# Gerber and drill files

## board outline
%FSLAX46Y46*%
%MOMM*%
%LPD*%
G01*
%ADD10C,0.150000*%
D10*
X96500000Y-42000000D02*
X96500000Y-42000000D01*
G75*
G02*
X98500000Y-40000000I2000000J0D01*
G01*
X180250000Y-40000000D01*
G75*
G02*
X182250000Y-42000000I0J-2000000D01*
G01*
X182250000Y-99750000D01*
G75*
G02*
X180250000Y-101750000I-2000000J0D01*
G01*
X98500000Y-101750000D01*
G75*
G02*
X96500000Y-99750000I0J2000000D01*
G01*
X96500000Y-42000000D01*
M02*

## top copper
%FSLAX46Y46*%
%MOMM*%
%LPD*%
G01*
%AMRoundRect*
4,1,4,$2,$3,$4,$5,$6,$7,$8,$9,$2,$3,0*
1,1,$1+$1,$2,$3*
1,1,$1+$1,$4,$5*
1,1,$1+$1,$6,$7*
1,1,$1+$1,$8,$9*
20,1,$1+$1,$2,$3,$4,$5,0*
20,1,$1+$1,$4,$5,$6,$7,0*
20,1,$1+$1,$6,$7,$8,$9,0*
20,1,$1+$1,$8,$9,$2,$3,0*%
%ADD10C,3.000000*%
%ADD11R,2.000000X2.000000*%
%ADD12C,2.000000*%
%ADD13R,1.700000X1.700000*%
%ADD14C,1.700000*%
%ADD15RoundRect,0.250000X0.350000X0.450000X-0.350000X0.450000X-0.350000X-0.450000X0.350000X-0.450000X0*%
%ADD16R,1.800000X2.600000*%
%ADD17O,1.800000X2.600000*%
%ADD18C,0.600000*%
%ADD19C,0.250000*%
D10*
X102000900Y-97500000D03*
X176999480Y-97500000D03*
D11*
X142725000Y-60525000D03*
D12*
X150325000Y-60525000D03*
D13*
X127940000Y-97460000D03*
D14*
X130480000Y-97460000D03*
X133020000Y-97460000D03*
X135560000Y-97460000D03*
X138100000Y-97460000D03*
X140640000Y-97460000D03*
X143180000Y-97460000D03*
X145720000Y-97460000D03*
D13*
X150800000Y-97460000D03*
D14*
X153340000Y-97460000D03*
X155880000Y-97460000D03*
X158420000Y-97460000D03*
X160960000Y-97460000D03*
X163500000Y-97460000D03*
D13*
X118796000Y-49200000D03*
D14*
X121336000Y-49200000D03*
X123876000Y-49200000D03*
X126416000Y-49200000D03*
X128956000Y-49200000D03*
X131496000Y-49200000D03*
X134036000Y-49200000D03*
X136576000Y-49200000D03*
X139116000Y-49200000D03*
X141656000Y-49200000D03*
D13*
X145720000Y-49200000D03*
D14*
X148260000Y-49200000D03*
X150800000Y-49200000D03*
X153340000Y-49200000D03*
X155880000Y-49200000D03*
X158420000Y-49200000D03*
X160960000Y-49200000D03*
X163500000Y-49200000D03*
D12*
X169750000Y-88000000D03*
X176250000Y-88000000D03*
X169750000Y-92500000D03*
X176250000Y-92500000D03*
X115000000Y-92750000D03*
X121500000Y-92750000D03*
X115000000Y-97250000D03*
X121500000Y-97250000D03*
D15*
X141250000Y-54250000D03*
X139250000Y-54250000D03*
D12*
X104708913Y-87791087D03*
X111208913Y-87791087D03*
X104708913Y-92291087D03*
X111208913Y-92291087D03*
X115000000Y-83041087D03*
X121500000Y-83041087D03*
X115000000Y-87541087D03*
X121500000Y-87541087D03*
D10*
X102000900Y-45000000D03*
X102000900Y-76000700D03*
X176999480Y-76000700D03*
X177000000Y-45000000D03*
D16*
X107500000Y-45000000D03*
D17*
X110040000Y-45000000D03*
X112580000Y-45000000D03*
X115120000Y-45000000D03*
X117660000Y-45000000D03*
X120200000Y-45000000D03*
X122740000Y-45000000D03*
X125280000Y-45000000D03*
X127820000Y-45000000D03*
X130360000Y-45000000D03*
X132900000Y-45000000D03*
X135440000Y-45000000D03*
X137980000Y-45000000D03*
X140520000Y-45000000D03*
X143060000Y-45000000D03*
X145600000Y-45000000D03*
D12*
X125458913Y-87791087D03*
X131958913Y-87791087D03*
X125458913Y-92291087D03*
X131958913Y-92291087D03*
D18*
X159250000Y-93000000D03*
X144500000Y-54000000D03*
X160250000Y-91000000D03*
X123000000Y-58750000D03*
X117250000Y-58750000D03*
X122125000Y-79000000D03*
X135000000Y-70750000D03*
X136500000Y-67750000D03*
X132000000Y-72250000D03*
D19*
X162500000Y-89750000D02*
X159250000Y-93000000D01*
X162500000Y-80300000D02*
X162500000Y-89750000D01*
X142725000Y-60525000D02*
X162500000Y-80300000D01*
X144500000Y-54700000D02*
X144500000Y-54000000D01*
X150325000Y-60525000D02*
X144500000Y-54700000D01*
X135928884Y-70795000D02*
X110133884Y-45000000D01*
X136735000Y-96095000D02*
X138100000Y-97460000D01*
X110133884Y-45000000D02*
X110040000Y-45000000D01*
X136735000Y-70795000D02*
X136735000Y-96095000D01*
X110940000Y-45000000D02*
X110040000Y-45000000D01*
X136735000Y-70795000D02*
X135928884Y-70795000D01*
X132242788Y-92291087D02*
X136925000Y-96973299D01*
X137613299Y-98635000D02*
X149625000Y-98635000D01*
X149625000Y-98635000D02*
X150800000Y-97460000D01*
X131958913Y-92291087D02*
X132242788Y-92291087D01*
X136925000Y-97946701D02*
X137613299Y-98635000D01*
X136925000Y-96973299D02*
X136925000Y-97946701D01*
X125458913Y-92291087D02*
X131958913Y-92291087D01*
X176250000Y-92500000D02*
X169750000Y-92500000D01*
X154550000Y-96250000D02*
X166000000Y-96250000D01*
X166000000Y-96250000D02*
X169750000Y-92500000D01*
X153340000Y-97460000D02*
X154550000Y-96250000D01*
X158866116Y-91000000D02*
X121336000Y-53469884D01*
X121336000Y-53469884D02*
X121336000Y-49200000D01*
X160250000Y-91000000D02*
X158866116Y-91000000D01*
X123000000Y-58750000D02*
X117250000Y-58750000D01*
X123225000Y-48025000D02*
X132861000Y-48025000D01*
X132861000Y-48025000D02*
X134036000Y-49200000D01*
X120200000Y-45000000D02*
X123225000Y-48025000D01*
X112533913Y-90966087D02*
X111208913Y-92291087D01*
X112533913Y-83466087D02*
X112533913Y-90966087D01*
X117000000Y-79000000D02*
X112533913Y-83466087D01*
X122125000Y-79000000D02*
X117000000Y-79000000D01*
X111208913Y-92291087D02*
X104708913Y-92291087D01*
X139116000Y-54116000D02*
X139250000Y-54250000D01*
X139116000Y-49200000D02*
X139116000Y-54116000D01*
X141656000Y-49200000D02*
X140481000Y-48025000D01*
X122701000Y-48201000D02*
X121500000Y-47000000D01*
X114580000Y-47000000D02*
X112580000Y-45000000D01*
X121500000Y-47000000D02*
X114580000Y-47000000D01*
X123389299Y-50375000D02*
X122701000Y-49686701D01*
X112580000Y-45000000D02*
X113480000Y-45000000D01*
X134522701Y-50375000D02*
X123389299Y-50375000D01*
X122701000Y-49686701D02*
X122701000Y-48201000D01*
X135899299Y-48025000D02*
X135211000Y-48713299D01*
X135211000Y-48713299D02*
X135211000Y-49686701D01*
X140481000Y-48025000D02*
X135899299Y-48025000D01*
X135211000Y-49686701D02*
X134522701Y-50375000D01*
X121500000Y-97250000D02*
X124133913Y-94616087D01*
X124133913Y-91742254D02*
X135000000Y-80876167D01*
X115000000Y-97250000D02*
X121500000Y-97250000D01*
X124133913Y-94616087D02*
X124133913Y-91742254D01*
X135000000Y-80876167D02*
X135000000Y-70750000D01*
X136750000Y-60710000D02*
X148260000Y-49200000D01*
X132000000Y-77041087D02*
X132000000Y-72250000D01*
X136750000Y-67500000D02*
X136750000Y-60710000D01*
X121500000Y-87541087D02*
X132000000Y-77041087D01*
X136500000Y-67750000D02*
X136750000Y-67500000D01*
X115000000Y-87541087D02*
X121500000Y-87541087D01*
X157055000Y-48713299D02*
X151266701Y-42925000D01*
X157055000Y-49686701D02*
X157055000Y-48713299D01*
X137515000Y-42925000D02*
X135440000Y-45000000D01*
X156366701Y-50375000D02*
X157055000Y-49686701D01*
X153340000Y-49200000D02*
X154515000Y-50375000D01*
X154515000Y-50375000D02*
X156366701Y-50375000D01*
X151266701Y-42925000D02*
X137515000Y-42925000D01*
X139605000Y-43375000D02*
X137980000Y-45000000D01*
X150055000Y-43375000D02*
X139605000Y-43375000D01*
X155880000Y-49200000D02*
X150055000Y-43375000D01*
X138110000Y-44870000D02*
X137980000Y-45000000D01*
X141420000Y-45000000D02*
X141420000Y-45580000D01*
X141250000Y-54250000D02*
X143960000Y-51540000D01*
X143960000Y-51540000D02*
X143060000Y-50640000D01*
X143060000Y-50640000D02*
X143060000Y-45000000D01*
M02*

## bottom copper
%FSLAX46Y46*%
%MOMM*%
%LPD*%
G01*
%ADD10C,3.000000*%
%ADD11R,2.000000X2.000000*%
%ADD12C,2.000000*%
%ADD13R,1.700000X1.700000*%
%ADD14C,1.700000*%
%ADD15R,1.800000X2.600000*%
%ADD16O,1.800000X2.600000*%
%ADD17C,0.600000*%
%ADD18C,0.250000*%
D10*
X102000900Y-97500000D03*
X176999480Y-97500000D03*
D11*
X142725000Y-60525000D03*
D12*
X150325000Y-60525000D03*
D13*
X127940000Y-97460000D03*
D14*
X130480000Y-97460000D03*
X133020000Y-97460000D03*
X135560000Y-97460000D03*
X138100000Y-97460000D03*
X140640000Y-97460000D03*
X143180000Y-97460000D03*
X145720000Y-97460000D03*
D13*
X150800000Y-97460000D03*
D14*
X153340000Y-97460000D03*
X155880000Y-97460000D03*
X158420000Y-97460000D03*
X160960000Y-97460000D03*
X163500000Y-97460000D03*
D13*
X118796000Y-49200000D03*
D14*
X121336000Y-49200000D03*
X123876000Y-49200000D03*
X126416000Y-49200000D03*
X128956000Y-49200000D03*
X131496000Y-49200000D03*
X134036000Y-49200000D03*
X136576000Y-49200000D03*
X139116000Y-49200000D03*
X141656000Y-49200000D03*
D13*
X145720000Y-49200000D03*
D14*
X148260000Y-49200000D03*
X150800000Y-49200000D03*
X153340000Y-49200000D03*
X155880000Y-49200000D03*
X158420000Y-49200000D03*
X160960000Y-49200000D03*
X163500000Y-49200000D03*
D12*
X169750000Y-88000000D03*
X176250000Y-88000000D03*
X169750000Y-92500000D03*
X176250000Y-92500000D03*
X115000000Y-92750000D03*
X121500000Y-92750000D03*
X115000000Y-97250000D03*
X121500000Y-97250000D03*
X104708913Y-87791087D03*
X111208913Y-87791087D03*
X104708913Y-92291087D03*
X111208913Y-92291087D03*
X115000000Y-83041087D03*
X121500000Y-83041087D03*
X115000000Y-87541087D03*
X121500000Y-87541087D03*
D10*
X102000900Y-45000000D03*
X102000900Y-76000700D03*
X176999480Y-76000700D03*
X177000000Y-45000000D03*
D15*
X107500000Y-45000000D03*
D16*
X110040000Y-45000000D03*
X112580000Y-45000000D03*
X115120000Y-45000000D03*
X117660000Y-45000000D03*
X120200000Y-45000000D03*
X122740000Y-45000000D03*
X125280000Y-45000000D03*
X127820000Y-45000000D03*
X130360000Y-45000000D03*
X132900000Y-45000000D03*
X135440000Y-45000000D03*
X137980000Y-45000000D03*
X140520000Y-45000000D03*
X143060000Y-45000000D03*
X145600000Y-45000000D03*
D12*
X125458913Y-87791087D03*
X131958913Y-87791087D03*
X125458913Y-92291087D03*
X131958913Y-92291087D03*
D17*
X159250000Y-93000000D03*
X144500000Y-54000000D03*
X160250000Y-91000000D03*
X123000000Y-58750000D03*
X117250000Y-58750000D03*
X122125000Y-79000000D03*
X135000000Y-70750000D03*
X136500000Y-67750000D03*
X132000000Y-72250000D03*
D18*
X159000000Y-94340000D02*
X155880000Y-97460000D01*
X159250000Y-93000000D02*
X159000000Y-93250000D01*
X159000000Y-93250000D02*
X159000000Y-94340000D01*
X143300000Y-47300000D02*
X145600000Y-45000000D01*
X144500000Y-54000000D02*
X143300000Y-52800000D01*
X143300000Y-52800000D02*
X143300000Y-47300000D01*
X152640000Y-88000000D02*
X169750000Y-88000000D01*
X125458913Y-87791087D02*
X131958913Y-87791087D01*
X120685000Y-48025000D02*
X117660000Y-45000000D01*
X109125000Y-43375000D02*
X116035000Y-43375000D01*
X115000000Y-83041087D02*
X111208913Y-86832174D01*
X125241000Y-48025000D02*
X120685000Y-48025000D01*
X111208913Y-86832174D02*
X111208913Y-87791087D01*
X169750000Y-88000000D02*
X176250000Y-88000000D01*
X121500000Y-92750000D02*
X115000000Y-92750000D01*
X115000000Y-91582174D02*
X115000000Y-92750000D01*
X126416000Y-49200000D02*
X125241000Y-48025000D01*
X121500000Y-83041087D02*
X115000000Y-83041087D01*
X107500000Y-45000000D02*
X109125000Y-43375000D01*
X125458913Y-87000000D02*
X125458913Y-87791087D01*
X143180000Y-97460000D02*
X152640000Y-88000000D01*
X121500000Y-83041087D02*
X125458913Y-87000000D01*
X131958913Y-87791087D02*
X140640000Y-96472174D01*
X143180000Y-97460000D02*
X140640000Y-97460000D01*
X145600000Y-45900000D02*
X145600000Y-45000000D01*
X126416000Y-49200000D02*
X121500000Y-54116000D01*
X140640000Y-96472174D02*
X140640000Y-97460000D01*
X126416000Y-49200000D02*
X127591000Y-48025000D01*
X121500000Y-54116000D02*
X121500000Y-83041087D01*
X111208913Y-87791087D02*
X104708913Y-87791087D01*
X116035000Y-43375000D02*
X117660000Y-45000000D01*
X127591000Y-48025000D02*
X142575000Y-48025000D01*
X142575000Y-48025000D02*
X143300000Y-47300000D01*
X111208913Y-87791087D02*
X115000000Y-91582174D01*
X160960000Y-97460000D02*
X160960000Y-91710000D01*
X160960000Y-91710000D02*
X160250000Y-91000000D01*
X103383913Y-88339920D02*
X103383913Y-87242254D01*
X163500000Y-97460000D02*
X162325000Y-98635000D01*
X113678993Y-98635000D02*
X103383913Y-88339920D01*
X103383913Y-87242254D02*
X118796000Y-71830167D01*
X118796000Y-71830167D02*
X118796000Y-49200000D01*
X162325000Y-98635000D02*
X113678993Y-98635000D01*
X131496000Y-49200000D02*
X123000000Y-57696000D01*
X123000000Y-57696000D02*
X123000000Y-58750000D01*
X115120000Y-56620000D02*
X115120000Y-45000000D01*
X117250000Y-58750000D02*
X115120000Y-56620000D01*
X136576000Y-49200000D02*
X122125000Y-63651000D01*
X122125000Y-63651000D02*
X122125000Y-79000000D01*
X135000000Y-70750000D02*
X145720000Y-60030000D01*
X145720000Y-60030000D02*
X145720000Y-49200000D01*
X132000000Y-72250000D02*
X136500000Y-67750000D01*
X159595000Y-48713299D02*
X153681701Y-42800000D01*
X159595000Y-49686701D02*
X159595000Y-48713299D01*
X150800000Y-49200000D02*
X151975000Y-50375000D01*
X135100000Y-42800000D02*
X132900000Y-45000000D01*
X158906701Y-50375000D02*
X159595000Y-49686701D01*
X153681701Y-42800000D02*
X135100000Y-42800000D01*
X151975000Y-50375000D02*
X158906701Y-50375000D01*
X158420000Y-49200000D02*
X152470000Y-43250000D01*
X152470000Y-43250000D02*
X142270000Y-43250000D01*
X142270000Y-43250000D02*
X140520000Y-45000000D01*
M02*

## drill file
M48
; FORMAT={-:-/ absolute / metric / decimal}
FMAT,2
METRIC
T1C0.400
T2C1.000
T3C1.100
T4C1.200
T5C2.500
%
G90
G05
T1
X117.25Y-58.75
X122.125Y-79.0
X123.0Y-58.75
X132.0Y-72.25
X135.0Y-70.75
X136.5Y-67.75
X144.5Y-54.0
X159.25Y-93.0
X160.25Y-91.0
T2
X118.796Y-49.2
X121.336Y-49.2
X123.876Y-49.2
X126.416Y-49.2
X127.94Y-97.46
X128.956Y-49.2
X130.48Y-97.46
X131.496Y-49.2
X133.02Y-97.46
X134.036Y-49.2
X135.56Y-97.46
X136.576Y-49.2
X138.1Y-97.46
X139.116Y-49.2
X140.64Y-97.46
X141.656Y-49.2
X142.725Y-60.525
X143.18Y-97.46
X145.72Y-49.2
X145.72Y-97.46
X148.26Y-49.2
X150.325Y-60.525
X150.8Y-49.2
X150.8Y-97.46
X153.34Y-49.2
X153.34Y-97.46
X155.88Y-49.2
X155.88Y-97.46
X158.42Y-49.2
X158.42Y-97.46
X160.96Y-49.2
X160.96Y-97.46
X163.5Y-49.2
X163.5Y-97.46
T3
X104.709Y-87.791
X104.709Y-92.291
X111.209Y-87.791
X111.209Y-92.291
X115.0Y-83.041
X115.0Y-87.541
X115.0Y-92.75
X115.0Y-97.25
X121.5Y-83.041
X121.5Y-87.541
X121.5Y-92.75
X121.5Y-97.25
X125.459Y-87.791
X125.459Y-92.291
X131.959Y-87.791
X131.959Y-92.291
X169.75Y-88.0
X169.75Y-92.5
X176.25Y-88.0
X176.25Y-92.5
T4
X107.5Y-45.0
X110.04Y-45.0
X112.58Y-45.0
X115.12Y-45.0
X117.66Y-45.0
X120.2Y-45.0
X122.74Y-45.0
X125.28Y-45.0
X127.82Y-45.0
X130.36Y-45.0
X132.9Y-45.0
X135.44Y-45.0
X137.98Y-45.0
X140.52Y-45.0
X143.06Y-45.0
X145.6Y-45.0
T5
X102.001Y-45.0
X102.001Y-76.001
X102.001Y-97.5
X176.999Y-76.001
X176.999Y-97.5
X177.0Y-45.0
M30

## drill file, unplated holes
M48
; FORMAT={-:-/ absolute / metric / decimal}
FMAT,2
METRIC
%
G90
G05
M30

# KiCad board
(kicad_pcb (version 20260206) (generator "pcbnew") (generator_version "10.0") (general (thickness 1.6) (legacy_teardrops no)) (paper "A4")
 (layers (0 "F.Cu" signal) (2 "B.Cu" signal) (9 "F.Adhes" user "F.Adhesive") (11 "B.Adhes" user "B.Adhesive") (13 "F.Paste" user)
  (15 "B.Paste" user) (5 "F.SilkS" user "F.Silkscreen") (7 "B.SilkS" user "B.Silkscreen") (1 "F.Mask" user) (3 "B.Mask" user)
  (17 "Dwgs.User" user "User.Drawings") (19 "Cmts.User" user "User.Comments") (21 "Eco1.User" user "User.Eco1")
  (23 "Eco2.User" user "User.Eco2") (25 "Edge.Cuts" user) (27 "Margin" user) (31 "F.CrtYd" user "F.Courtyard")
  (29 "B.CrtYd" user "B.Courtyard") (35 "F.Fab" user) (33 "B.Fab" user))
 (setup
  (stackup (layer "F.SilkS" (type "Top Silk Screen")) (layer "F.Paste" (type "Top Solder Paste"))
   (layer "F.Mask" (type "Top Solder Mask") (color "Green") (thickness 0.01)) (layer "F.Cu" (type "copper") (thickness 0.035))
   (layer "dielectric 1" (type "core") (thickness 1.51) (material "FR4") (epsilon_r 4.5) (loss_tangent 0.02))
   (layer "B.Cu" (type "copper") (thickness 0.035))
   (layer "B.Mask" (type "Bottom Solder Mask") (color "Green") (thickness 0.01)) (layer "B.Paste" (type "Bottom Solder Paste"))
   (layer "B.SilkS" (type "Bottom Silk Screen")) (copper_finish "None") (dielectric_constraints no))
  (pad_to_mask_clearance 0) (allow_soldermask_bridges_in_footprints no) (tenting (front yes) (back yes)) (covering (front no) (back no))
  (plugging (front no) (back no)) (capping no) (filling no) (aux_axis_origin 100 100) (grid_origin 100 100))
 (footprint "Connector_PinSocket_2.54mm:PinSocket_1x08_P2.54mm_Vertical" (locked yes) (layer "F.Cu") (at 127.94 97.46 90)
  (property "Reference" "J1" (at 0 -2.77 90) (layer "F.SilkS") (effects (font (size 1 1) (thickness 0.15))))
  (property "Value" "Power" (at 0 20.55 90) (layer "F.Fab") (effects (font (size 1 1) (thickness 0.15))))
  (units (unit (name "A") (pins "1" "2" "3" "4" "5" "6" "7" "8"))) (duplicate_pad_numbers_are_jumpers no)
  (pad "1" thru_hole rect (at 0 0 90) (size 1.7 1.7) (drill 1) (layers "*.Cu" "*.Mask") (remove_unused_layers no)
   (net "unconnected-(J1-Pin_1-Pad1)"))
  (pad "2" thru_hole circle (at 0 2.54 90) (size 1.7 1.7) (drill 1) (layers "*.Cu" "*.Mask") (remove_unused_layers no) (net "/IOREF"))
  (pad "3" thru_hole circle (at 0 5.08 90) (size 1.7 1.7) (drill 1) (layers "*.Cu" "*.Mask") (remove_unused_layers no) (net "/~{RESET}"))
  (pad "4" thru_hole circle (at 0 7.62 90) (size 1.7 1.7) (drill 1) (layers "*.Cu" "*.Mask") (remove_unused_layers no) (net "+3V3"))
  (pad "5" thru_hole circle (at 0 10.16 90) (size 1.7 1.7) (drill 1) (layers "*.Cu" "*.Mask") (remove_unused_layers no) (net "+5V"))
  (pad "6" thru_hole circle (at 0 12.7 90) (size 1.7 1.7) (drill 1) (layers "*.Cu" "*.Mask") (remove_unused_layers no) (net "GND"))
  (pad "7" thru_hole circle (at 0 15.24 90) (size 1.7 1.7) (drill 1) (layers "*.Cu" "*.Mask") (remove_unused_layers no) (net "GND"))
  (pad "8" thru_hole circle (at 0 17.78 90) (size 1.7 1.7) (drill 1) (layers "*.Cu" "*.Mask") (remove_unused_layers no) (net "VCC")))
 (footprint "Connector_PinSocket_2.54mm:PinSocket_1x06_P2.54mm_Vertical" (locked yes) (layer "F.Cu") (at 150.8 97.46 90)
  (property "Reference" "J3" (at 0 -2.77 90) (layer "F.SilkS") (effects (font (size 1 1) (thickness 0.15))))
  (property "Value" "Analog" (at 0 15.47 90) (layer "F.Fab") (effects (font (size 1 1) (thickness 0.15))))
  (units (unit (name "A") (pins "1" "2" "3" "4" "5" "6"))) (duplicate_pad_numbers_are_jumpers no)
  (pad "1" thru_hole rect (at 0 0 90) (size 1.7 1.7) (drill 1) (layers "*.Cu" "*.Mask") (remove_unused_layers no) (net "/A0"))
  (pad "2" thru_hole circle (at 0 2.54 90) (size 1.7 1.7) (drill 1) (layers "*.Cu" "*.Mask") (remove_unused_layers no) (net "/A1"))
  (pad "3" thru_hole circle (at 0 5.08 90) (size 1.7 1.7) (drill 1) (layers "*.Cu" "*.Mask") (remove_unused_layers no) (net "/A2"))
  (pad "4" thru_hole circle (at 0 7.62 90) (size 1.7 1.7) (drill 1) (layers "*.Cu" "*.Mask") (remove_unused_layers no) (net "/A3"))
  (pad "5" thru_hole circle (at 0 10.16 90) (size 1.7 1.7) (drill 1) (layers "*.Cu" "*.Mask") (remove_unused_layers no)
   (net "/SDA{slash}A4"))
  (pad "6" thru_hole circle (at 0 12.7 90) (size 1.7 1.7) (drill 1) (layers "*.Cu" "*.Mask") (remove_unused_layers no) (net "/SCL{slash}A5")))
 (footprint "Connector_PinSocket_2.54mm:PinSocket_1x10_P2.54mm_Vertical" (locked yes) (layer "F.Cu") (at 118.796 49.2 90)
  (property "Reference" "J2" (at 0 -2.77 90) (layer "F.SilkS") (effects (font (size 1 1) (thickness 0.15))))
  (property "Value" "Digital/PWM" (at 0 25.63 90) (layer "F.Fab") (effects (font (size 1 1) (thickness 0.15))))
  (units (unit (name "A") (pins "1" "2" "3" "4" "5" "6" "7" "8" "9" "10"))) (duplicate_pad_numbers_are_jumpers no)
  (pad "1" thru_hole rect (at 0 0 90) (size 1.7 1.7) (drill 1) (layers "*.Cu" "*.Mask") (remove_unused_layers no) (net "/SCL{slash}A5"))
  (pad "2" thru_hole circle (at 0 2.54 90) (size 1.7 1.7) (drill 1) (layers "*.Cu" "*.Mask") (remove_unused_layers no) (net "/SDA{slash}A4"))
  (pad "3" thru_hole circle (at 0 5.08 90) (size 1.7 1.7) (drill 1) (layers "*.Cu" "*.Mask") (remove_unused_layers no) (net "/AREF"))
  (pad "4" thru_hole circle (at 0 7.62 90) (size 1.7 1.7) (drill 1) (layers "*.Cu" "*.Mask") (remove_unused_layers no) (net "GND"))
  (pad "5" thru_hole circle (at 0 10.16 90) (size 1.7 1.7) (drill 1) (layers "*.Cu" "*.Mask") (remove_unused_layers no) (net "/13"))
  (pad "6" thru_hole circle (at 0 12.7 90) (size 1.7 1.7) (drill 1) (layers "*.Cu" "*.Mask") (remove_unused_layers no) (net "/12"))
  (pad "7" thru_hole circle (at 0 15.24 90) (size 1.7 1.7) (drill 1) (layers "*.Cu" "*.Mask") (remove_unused_layers no) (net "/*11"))
  (pad "8" thru_hole circle (at 0 17.78 90) (size 1.7 1.7) (drill 1) (layers "*.Cu" "*.Mask") (remove_unused_layers no) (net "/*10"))
  (pad "9" thru_hole circle (at 0 20.32 90) (size 1.7 1.7) (drill 1) (layers "*.Cu" "*.Mask") (remove_unused_layers no) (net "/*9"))
  (pad "10" thru_hole circle (at 0 22.86 90) (size 1.7 1.7) (drill 1) (layers "*.Cu" "*.Mask") (remove_unused_layers no) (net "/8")))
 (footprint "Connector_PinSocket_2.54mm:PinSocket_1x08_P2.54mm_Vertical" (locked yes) (layer "F.Cu") (at 145.72 49.2 90)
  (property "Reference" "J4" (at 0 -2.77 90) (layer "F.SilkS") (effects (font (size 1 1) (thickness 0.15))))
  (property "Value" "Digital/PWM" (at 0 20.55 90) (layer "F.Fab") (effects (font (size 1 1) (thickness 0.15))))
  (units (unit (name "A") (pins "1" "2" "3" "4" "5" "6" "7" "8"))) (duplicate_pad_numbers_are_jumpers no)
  (pad "1" thru_hole rect (at 0 0 90) (size 1.7 1.7) (drill 1) (layers "*.Cu" "*.Mask") (remove_unused_layers no) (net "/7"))
  (pad "2" thru_hole circle (at 0 2.54 90) (size 1.7 1.7) (drill 1) (layers "*.Cu" "*.Mask") (remove_unused_layers no) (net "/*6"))
  (pad "3" thru_hole circle (at 0 5.08 90) (size 1.7 1.7) (drill 1) (layers "*.Cu" "*.Mask") (remove_unused_layers no) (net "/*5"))
  (pad "4" thru_hole circle (at 0 7.62 90) (size 1.7 1.7) (drill 1) (layers "*.Cu" "*.Mask") (remove_unused_layers no) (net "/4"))
  (pad "5" thru_hole circle (at 0 10.16 90) (size 1.7 1.7) (drill 1) (layers "*.Cu" "*.Mask") (remove_unused_layers no) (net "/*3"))
  (pad "6" thru_hole circle (at 0 12.7 90) (size 1.7 1.7) (drill 1) (layers "*.Cu" "*.Mask") (remove_unused_layers no) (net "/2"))
  (pad "7" thru_hole circle (at 0 15.24 90) (size 1.7 1.7) (drill 1) (layers "*.Cu" "*.Mask") (remove_unused_layers no) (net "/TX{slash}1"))
  (pad "8" thru_hole circle (at 0 17.78 90) (size 1.7 1.7) (drill 1) (layers "*.Cu" "*.Mask") (remove_unused_layers no) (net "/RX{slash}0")))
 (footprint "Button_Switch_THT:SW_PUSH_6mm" (layer "F.Cu") (at 169.75 88)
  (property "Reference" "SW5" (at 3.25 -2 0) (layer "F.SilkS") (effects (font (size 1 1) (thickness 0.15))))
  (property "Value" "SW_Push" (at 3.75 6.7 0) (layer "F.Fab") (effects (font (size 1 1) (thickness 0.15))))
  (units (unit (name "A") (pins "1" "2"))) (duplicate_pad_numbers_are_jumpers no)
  (pad "1" thru_hole circle (at 0 0 90) (size 2 2) (drill 1.1) (layers "*.Cu" "*.Mask") (remove_unused_layers no) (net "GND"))
  (pad "1" thru_hole circle (at 6.5 0 90) (size 2 2) (drill 1.1) (layers "*.Cu" "*.Mask") (remove_unused_layers no) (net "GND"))
  (pad "2" thru_hole circle (at 0 4.5 90) (size 2 2) (drill 1.1) (layers "*.Cu" "*.Mask") (remove_unused_layers no) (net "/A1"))
  (pad "2" thru_hole circle (at 6.5 4.5 90) (size 2 2) (drill 1.1) (layers "*.Cu" "*.Mask") (remove_unused_layers no) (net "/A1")))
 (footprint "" (layer "F.Cu") (at 176.99948 97.5)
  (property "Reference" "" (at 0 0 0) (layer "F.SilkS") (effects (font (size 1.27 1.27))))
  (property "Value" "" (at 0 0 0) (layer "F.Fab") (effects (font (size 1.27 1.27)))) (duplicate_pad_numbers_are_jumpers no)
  (pad "" thru_hole circle (at 0 0) (size 3 3) (drill 2.5) (layers "*.Cu" "*.Mask") (remove_unused_layers no)))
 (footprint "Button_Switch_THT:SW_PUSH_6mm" (layer "F.Cu") (at 115 92.75)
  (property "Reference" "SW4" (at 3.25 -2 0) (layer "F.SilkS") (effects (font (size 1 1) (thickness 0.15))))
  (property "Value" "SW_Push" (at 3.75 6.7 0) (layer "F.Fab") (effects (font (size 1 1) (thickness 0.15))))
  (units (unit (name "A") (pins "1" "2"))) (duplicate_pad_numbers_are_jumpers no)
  (pad "1" thru_hole circle (at 0 0 90) (size 2 2) (drill 1.1) (layers "*.Cu" "*.Mask") (remove_unused_layers no) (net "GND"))
  (pad "1" thru_hole circle (at 6.5 0 90) (size 2 2) (drill 1.1) (layers "*.Cu" "*.Mask") (remove_unused_layers no) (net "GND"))
  (pad "2" thru_hole circle (at 0 4.5 90) (size 2 2) (drill 1.1) (layers "*.Cu" "*.Mask") (remove_unused_layers no) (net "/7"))
  (pad "2" thru_hole circle (at 6.5 4.5 90) (size 2 2) (drill 1.1) (layers "*.Cu" "*.Mask") (remove_unused_layers no) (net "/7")))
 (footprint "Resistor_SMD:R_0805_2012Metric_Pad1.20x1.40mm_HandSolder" (layer "F.Cu") (at 140.25 54.25 180)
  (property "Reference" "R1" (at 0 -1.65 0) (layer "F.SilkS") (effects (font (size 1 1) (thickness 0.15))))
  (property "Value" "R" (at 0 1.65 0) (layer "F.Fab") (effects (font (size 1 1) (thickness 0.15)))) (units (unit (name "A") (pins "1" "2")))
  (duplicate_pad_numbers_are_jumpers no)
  (pad "1" smd roundrect (at -1 0 180) (size 1.2 1.4) (layers "F.Cu" "F.Mask" "F.Paste") (roundrect_rratio 0.208333)
   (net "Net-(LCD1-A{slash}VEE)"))
  (pad "2" smd roundrect (at 1 0 180) (size 1.2 1.4) (layers "F.Cu" "F.Mask" "F.Paste") (roundrect_rratio 0.208333) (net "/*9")))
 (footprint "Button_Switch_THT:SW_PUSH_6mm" (layer "F.Cu") (at 104.708913 87.791087)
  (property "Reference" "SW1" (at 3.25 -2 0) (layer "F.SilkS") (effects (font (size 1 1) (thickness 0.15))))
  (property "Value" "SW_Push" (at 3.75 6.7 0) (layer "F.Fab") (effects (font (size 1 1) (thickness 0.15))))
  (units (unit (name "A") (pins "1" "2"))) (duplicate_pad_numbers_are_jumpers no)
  (pad "1" thru_hole circle (at 0 0 90) (size 2 2) (drill 1.1) (layers "*.Cu" "*.Mask") (remove_unused_layers no) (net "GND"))
  (pad "1" thru_hole circle (at 6.5 0 90) (size 2 2) (drill 1.1) (layers "*.Cu" "*.Mask") (remove_unused_layers no) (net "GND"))
  (pad "2" thru_hole circle (at 0 4.5 90) (size 2 2) (drill 1.1) (layers "*.Cu" "*.Mask") (remove_unused_layers no) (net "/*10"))
  (pad "2" thru_hole circle (at 6.5 4.5 90) (size 2 2) (drill 1.1) (layers "*.Cu" "*.Mask") (remove_unused_layers no) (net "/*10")))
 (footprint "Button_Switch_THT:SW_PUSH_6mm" (layer "F.Cu") (at 115 83.041087)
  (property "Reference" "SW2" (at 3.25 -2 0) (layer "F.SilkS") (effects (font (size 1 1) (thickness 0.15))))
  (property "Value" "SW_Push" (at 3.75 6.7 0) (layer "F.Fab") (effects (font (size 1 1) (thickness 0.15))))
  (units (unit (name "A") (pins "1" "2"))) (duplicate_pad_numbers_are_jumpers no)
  (pad "1" thru_hole circle (at 0 0 90) (size 2 2) (drill 1.1) (layers "*.Cu" "*.Mask") (remove_unused_layers no) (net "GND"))
  (pad "1" thru_hole circle (at 6.5 0 90) (size 2 2) (drill 1.1) (layers "*.Cu" "*.Mask") (remove_unused_layers no) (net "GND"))
  (pad "2" thru_hole circle (at 0 4.5 90) (size 2 2) (drill 1.1) (layers "*.Cu" "*.Mask") (remove_unused_layers no) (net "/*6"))
  (pad "2" thru_hole circle (at 6.5 4.5 90) (size 2 2) (drill 1.1) (layers "*.Cu" "*.Mask") (remove_unused_layers no) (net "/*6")))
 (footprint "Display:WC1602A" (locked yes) (layer "F.Cu") (at 107.5 45)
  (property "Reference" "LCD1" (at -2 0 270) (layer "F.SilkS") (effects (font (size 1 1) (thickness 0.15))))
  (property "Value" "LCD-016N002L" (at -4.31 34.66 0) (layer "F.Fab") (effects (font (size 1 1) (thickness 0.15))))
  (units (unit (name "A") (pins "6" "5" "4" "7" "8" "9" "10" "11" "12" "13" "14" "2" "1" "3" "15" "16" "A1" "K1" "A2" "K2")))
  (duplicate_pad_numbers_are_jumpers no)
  (pad "" thru_hole circle (at -5.4991 0) (size 3 3) (drill 2.5) (layers "*.Cu" "*.Mask") (remove_unused_layers no))
  (pad "" thru_hole circle (at -5.4991 31.0007) (size 3 3) (drill 2.5) (layers "*.Cu" "*.Mask") (remove_unused_layers no))
  (pad "" thru_hole circle (at 69.49948 31.0007) (size 3 3) (drill 2.5) (layers "*.Cu" "*.Mask") (remove_unused_layers no))
  (pad "" thru_hole circle (at 69.5 0) (size 3 3) (drill 2.5) (layers "*.Cu" "*.Mask") (remove_unused_layers no))
  (pad "1" thru_hole rect (at 0 0) (size 1.8 2.6) (drill 1.2) (layers "*.Cu" "*.Mask") (remove_unused_layers no) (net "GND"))
  (pad "2" thru_hole oval (at 2.54 0) (size 1.8 2.6) (drill 1.2) (layers "*.Cu" "*.Mask") (remove_unused_layers no) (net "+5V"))
  (pad "3" thru_hole oval (at 5.08 0) (size 1.8 2.6) (drill 1.2) (layers "*.Cu" "*.Mask") (remove_unused_layers no) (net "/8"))
  (pad "4" thru_hole oval (at 7.62 0) (size 1.8 2.6) (drill 1.2) (layers "*.Cu" "*.Mask") (remove_unused_layers no) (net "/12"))
  (pad "5" thru_hole oval (at 10.16 0) (size 1.8 2.6) (drill 1.2) (layers "*.Cu" "*.Mask") (remove_unused_layers no) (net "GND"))
  (pad "6" thru_hole oval (at 12.7 0) (size 1.8 2.6) (drill 1.2) (layers "*.Cu" "*.Mask") (remove_unused_layers no) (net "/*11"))
  (pad "7" thru_hole oval (at 15.24 0) (size 1.8 2.6) (drill 1.2) (layers "*.Cu" "*.Mask") (remove_unused_layers no)
   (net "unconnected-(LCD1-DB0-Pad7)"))
  (pad "8" thru_hole oval (at 17.78 0) (size 1.8 2.6) (drill 1.2) (layers "*.Cu" "*.Mask") (remove_unused_layers no)
   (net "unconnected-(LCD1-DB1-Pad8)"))
  (pad "9" thru_hole oval (at 20.32 0) (size 1.8 2.6) (drill 1.2) (layers "*.Cu" "*.Mask") (remove_unused_layers no)
   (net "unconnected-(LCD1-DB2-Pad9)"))
  (pad "10" thru_hole oval (at 22.86 0) (size 1.8 2.6) (drill 1.2) (layers "*.Cu" "*.Mask") (remove_unused_layers no)
   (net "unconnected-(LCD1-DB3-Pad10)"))
  (pad "11" thru_hole oval (at 25.4 0) (size 1.8 2.6) (drill 1.2) (layers "*.Cu" "*.Mask") (remove_unused_layers no) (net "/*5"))
  (pad "12" thru_hole oval (at 27.94 0) (size 1.8 2.6) (drill 1.2) (layers "*.Cu" "*.Mask") (remove_unused_layers no) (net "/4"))
  (pad "13" thru_hole oval (at 30.48 0) (size 1.8 2.6) (drill 1.2) (layers "*.Cu" "*.Mask") (remove_unused_layers no) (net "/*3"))
  (pad "14" thru_hole oval (at 33.02 0) (size 1.8 2.6) (drill 1.2) (layers "*.Cu" "*.Mask") (remove_unused_layers no) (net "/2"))
  (pad "15" thru_hole oval (at 35.56 0) (size 1.8 2.6) (drill 1.2) (layers "*.Cu" "*.Mask") (remove_unused_layers no)
   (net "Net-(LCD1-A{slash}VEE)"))
  (pad "16" thru_hole oval (at 38.1 0) (size 1.8 2.6) (drill 1.2) (layers "*.Cu" "*.Mask") (remove_unused_layers no) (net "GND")))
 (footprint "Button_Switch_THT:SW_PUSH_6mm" (layer "F.Cu") (at 125.458913 87.791087)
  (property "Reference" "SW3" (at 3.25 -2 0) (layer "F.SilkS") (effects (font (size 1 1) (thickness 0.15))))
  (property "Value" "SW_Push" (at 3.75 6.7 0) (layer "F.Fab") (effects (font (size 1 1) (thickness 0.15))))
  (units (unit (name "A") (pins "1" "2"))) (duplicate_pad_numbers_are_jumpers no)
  (pad "1" thru_hole circle (at 0 0 90) (size 2 2) (drill 1.1) (layers "*.Cu" "*.Mask") (remove_unused_layers no) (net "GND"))
  (pad "1" thru_hole circle (at 6.5 0 90) (size 2 2) (drill 1.1) (layers "*.Cu" "*.Mask") (remove_unused_layers no) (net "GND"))
  (pad "2" thru_hole circle (at 0 4.5 90) (size 2 2) (drill 1.1) (layers "*.Cu" "*.Mask") (remove_unused_layers no) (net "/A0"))
  (pad "2" thru_hole circle (at 6.5 4.5 90) (size 2 2) (drill 1.1) (layers "*.Cu" "*.Mask") (remove_unused_layers no) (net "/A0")))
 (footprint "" (layer "F.Cu") (at 102.0009 97.5)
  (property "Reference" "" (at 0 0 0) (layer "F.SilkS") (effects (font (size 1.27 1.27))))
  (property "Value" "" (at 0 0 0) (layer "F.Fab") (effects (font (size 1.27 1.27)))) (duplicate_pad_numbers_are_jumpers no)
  (pad "" thru_hole circle (at 0 0) (size 3 3) (drill 2.5) (layers "*.Cu" "*.Mask") (remove_unused_layers no)))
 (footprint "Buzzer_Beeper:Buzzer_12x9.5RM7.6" (layer "F.Cu") (at 142.725 60.525)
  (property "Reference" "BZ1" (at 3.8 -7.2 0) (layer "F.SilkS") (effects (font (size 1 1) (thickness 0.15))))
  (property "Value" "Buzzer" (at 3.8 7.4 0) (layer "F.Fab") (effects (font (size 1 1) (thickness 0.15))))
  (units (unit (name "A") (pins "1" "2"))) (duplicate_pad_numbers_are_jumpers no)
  (pad "1" thru_hole rect (at 0 0) (size 2 2) (drill 1) (layers "*.Cu" "*.Mask") (remove_unused_layers no) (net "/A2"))
  (pad "2" thru_hole circle (at 7.6 0) (size 2 2) (drill 1) (layers "*.Cu" "*.Mask") (remove_unused_layers no) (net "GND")))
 (gr_rect (start 96.5 40) (end 182.25 101.75) (radius 2) (stroke (width 0.15) (type solid)) (fill no) (layer "Edge.Cuts"))
 (segment (start 135.928884 70.795) (end 110.133884 45) (width 0.25) (layer "F.Cu") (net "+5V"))
 (segment (start 136.735 96.095) (end 138.1 97.46) (width 0.25) (layer "F.Cu") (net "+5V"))
 (segment (start 110.133884 45) (end 110.04 45) (width 0.25) (layer "F.Cu") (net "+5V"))
 (segment (start 136.735 70.795) (end 136.735 96.095) (width 0.25) (layer "F.Cu") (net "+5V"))
 (segment (start 110.94 45) (end 110.04 45) (width 0.25) (layer "F.Cu") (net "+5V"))
 (segment (start 136.735 70.795) (end 135.928884 70.795) (width 0.25) (layer "F.Cu") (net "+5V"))
 (segment (start 144.5 54.7) (end 144.5 54) (width 0.25) (layer "F.Cu") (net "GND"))
 (segment (start 150.325 60.525) (end 144.5 54.7) (width 0.25) (layer "F.Cu") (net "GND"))
 (via (at 144.5 54) (size 0.6) (drill 0.4) (layers "F.Cu" "B.Cu") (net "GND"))
 (segment (start 143.3 47.3) (end 145.6 45) (width 0.25) (layer "B.Cu") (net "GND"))
 (segment (start 152.64 88) (end 169.75 88) (width 0.25) (layer "B.Cu") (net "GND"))
 (segment (start 125.458913 87.791087) (end 131.958913 87.791087) (width 0.25) (layer "B.Cu") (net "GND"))
 (segment (start 120.685 48.025) (end 117.66 45) (width 0.25) (layer "B.Cu") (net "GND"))
 (segment (start 109.125 43.375) (end 116.035 43.375) (width 0.25) (layer "B.Cu") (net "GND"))
 (segment (start 115 83.041087) (end 111.208913 86.832174) (width 0.25) (layer "B.Cu") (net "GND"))
 (segment (start 125.241 48.025) (end 120.685 48.025) (width 0.25) (layer "B.Cu") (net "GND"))
 (segment (start 111.208913 86.832174) (end 111.208913 87.791087) (width 0.25) (layer "B.Cu") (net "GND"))
 (segment (start 169.75 88) (end 176.25 88) (width 0.25) (layer "B.Cu") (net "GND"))
 (segment (start 121.5 92.75) (end 115 92.75) (width 0.25) (layer "B.Cu") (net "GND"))
 (segment (start 115 91.582174) (end 115 92.75) (width 0.25) (layer "B.Cu") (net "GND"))
 (segment (start 126.416 49.2) (end 125.241 48.025) (width 0.25) (layer "B.Cu") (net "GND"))
 (segment (start 121.5 83.041087) (end 115 83.041087) (width 0.25) (layer "B.Cu") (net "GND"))
 (segment (start 144.5 54) (end 143.3 52.8) (width 0.25) (layer "B.Cu") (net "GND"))
 (segment (start 107.5 45) (end 109.125 43.375) (width 0.25) (layer "B.Cu") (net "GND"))
 (segment (start 125.458913 87) (end 125.458913 87.791087) (width 0.25) (layer "B.Cu") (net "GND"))
 (segment (start 143.18 97.46) (end 152.64 88) (width 0.25) (layer "B.Cu") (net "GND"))
 (segment (start 121.5 83.041087) (end 125.458913 87) (width 0.25) (layer "B.Cu") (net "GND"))
 (segment (start 131.958913 87.791087) (end 140.64 96.472174) (width 0.25) (layer "B.Cu") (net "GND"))
 (segment (start 143.18 97.46) (end 140.64 97.46) (width 0.25) (layer "B.Cu") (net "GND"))
 (segment (start 145.6 45.9) (end 145.6 45) (width 0.25) (layer "B.Cu") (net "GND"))
 (segment (start 126.416 49.2) (end 121.5 54.116) (width 0.25) (layer "B.Cu") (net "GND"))
 (segment (start 140.64 96.472174) (end 140.64 97.46) (width 0.25) (layer "B.Cu") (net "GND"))
 (segment (start 126.416 49.2) (end 127.591 48.025) (width 0.25) (layer "B.Cu") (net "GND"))
 (segment (start 121.5 54.116) (end 121.5 83.041087) (width 0.25) (layer "B.Cu") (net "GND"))
 (segment (start 111.208913 87.791087) (end 104.708913 87.791087) (width 0.25) (layer "B.Cu") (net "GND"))
 (segment (start 143.3 52.8) (end 143.3 47.3) (width 0.25) (layer "B.Cu") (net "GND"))
 (segment (start 116.035 43.375) (end 117.66 45) (width 0.25) (layer "B.Cu") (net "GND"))
 (segment (start 127.591 48.025) (end 142.575 48.025) (width 0.25) (layer "B.Cu") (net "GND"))
 (segment (start 142.575 48.025) (end 143.3 47.3) (width 0.25) (layer "B.Cu") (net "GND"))
 (segment (start 111.208913 87.791087) (end 115 91.582174) (width 0.25) (layer "B.Cu") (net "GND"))
 (segment (start 132.242788 92.291087) (end 136.925 96.973299) (width 0.25) (layer "F.Cu") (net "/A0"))
 (segment (start 137.613299 98.635) (end 149.625 98.635) (width 0.25) (layer "F.Cu") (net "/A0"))
 (segment (start 149.625 98.635) (end 150.8 97.46) (width 0.25) (layer "F.Cu") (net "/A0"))
 (segment (start 131.958913 92.291087) (end 132.242788 92.291087) (width 0.25) (layer "F.Cu") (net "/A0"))
 (segment (start 136.925 97.946701) (end 137.613299 98.635) (width 0.25) (layer "F.Cu") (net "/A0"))
 (segment (start 136.925 96.973299) (end 136.925 97.946701) (width 0.25) (layer "F.Cu") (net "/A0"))
 (segment (start 125.458913 92.291087) (end 131.958913 92.291087) (width 0.25) (layer "F.Cu") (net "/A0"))
 (segment (start 176.25 92.5) (end 169.75 92.5) (width 0.25) (layer "F.Cu") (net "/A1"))
 (segment (start 154.55 96.25) (end 166 96.25) (width 0.25) (layer "F.Cu") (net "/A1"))
 (segment (start 166 96.25) (end 169.75 92.5) (width 0.25) (layer "F.Cu") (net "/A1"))
 (segment (start 153.34 97.46) (end 154.55 96.25) (width 0.25) (layer "F.Cu") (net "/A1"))
 (segment (start 162.5 89.75) (end 159.25 93) (width 0.25) (layer "F.Cu") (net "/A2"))
 (segment (start 162.5 80.3) (end 162.5 89.75) (width 0.25) (layer "F.Cu") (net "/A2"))
 (segment (start 142.725 60.525) (end 162.5 80.3) (width 0.25) (layer "F.Cu") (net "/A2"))
 (via (at 159.25 93) (size 0.6) (drill 0.4) (layers "F.Cu" "B.Cu") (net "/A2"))
 (segment (start 159.25 93) (end 159 93.25) (width 0.25) (layer "B.Cu") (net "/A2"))
 (segment (start 159 93.25) (end 159 94.34) (width 0.25) (layer "B.Cu") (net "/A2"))
 (segment (start 159 94.34) (end 155.88 97.46) (width 0.25) (layer "B.Cu") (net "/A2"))
 (segment (start 158.866116 91) (end 121.336 53.469884) (width 0.25) (layer "F.Cu") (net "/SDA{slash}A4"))
 (segment (start 121.336 53.469884) (end 121.336 49.2) (width 0.25) (layer "F.Cu") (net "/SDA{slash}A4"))
 (segment (start 160.25 91) (end 158.866116 91) (width 0.25) (layer "F.Cu") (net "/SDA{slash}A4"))
 (via (at 160.25 91) (size 0.6) (drill 0.4) (layers "F.Cu" "B.Cu") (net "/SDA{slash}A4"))
 (segment (start 160.96 97.46) (end 160.96 91.71) (width 0.25) (layer "B.Cu") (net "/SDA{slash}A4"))
 (segment (start 160.96 91.71) (end 160.25 91) (width 0.25) (layer "B.Cu") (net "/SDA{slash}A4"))
 (segment (start 103.383913 88.33992) (end 103.383913 87.242254) (width 0.25) (layer "B.Cu") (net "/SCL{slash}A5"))
 (segment (start 163.5 97.46) (end 162.325 98.635) (width 0.25) (layer "B.Cu") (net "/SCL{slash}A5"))
 (segment (start 113.678993 98.635) (end 103.383913 88.33992) (width 0.25) (layer "B.Cu") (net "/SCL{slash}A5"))
 (segment (start 103.383913 87.242254) (end 118.796 71.830167) (width 0.25) (layer "B.Cu") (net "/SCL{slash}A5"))
 (segment (start 118.796 71.830167) (end 118.796 49.2) (width 0.25) (layer "B.Cu") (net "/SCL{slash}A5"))
 (segment (start 162.325 98.635) (end 113.678993 98.635) (width 0.25) (layer "B.Cu") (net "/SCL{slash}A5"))
 (segment (start 123 58.75) (end 117.25 58.75) (width 0.25) (layer "F.Cu") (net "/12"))
 (via (at 123 58.75) (size 0.6) (drill 0.4) (layers "F.Cu" "B.Cu") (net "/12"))
 (via (at 117.25 58.75) (size 0.6) (drill 0.4) (layers "F.Cu" "B.Cu") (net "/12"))
 (segment (start 131.496 49.2) (end 123 57.696) (width 0.25) (layer "B.Cu") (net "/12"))
 (segment (start 123 57.696) (end 123 58.75) (width 0.25) (layer "B.Cu") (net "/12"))
 (segment (start 115.12 56.62) (end 115.12 45) (width 0.25) (layer "B.Cu") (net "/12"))
 (segment (start 117.25 58.75) (end 115.12 56.62) (width 0.25) (layer "B.Cu") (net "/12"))
 (segment (start 123.225 48.025) (end 132.861 48.025) (width 0.25) (layer "F.Cu") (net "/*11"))
 (segment (start 132.861 48.025) (end 134.036 49.2) (width 0.25) (layer "F.Cu") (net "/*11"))
 (segment (start 120.2 45) (end 123.225 48.025) (width 0.25) (layer "F.Cu") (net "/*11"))
 (segment (start 112.533913 90.966087) (end 111.208913 92.291087) (width 0.25) (layer "F.Cu") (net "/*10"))
 (segment (start 112.533913 83.466087) (end 112.533913 90.966087) (width 0.25) (layer "F.Cu") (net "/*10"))
 (segment (start 117 79) (end 112.533913 83.466087) (width 0.25) (layer "F.Cu") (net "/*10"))
 (segment (start 122.125 79) (end 117 79) (width 0.25) (layer "F.Cu") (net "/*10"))
 (segment (start 111.208913 92.291087) (end 104.708913 92.291087) (width 0.25) (layer "F.Cu") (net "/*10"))
 (via (at 122.125 79) (size 0.6) (drill 0.4) (layers "F.Cu" "B.Cu") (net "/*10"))
 (segment (start 136.576 49.2) (end 122.125 63.651) (width 0.25) (layer "B.Cu") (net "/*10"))
 (segment (start 122.125 63.651) (end 122.125 79) (width 0.25) (layer "B.Cu") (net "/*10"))
 (segment (start 139.116 54.116) (end 139.25 54.25) (width 0.25) (layer "F.Cu") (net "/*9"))
 (segment (start 139.116 49.2) (end 139.116 54.116) (width 0.25) (layer "F.Cu") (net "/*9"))
 (segment (start 141.656 49.2) (end 140.481 48.025) (width 0.25) (layer "F.Cu") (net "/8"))
 (segment (start 122.701 48.201) (end 121.5 47) (width 0.25) (layer "F.Cu") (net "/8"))
 (segment (start 114.58 47) (end 112.58 45) (width 0.25) (layer "F.Cu") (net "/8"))
 (segment (start 121.5 47) (end 114.58 47) (width 0.25) (layer "F.Cu") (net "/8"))
 (segment (start 123.389299 50.375) (end 122.701 49.686701) (width 0.25) (layer "F.Cu") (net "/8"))
 (segment (start 112.58 45) (end 113.48 45) (width 0.25) (layer "F.Cu") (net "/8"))
 (segment (start 134.522701 50.375) (end 123.389299 50.375) (width 0.25) (layer "F.Cu") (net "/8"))
 (segment (start 122.701 49.686701) (end 122.701 48.201) (width 0.25) (layer "F.Cu") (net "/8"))
 (segment (start 135.899299 48.025) (end 135.211 48.713299) (width 0.25) (layer "F.Cu") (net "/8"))
 (segment (start 135.211 48.713299) (end 135.211 49.686701) (width 0.25) (layer "F.Cu") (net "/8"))
 (segment (start 140.481 48.025) (end 135.899299 48.025) (width 0.25) (layer "F.Cu") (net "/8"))
 (segment (start 135.211 49.686701) (end 134.522701 50.375) (width 0.25) (layer "F.Cu") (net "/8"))
 (segment (start 121.5 97.25) (end 124.133913 94.616087) (width 0.25) (layer "F.Cu") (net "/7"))
 (segment (start 124.133913 91.742254) (end 135 80.876167) (width 0.25) (layer "F.Cu") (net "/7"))
 (segment (start 115 97.25) (end 121.5 97.25) (width 0.25) (layer "F.Cu") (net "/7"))
 (segment (start 124.133913 94.616087) (end 124.133913 91.742254) (width 0.25) (layer "F.Cu") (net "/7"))
 (segment (start 135 80.876167) (end 135 70.75) (width 0.25) (layer "F.Cu") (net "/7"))
 (via (at 135 70.75) (size 0.6) (drill 0.4) (layers "F.Cu" "B.Cu") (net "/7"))
 (segment (start 135 70.75) (end 145.72 60.03) (width 0.25) (layer "B.Cu") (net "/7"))
 (segment (start 145.72 60.03) (end 145.72 49.2) (width 0.25) (layer "B.Cu") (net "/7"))
 (segment (start 136.75 60.71) (end 148.26 49.2) (width 0.25) (layer "F.Cu") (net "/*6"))
 (segment (start 132 77.041087) (end 132 72.25) (width 0.25) (layer "F.Cu") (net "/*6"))
 (segment (start 136.75 67.5) (end 136.75 60.71) (width 0.25) (layer "F.Cu") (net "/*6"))
 (segment (start 121.5 87.541087) (end 132 77.041087) (width 0.25) (layer "F.Cu") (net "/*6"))
 (segment (start 136.5 67.75) (end 136.75 67.5) (width 0.25) (layer "F.Cu") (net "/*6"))
 (segment (start 115 87.541087) (end 121.5 87.541087) (width 0.25) (layer "F.Cu") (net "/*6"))
 (via (at 136.5 67.75) (size 0.6) (drill 0.4) (layers "F.Cu" "B.Cu") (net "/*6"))
 (via (at 132 72.25) (size 0.6) (drill 0.4) (layers "F.Cu" "B.Cu") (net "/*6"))
 (segment (start 132 72.25) (end 136.5 67.75) (width 0.25) (layer "B.Cu") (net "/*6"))
 (segment (start 159.595 48.713299) (end 153.681701 42.8) (width 0.25) (layer "B.Cu") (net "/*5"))
 (segment (start 159.595 49.686701) (end 159.595 48.713299) (width 0.25) (layer "B.Cu") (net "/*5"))
 (segment (start 150.8 49.2) (end 151.975 50.375) (width 0.25) (layer "B.Cu") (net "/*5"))
 (segment (start 135.1 42.8) (end 132.9 45) (width 0.25) (layer "B.Cu") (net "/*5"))
 (segment (start 158.906701 50.375) (end 159.595 49.686701) (width 0.25) (layer "B.Cu") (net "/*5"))
 (segment (start 153.681701 42.8) (end 135.1 42.8) (width 0.25) (layer "B.Cu") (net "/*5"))
 (segment (start 151.975 50.375) (end 158.906701 50.375) (width 0.25) (layer "B.Cu") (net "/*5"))
 (segment (start 157.055 48.713299) (end 151.266701 42.925) (width 0.25) (layer "F.Cu") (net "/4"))
 (segment (start 157.055 49.686701) (end 157.055 48.713299) (width 0.25) (layer "F.Cu") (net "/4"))
 (segment (start 137.515 42.925) (end 135.44 45) (width 0.25) (layer "F.Cu") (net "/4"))
 (segment (start 156.366701 50.375) (end 157.055 49.686701) (width 0.25) (layer "F.Cu") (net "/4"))
 (segment (start 153.34 49.2) (end 154.515 50.375) (width 0.25) (layer "F.Cu") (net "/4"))
 (segment (start 154.515 50.375) (end 156.366701 50.375) (width 0.25) (layer "F.Cu") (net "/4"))
 (segment (start 151.266701 42.925) (end 137.515 42.925) (width 0.25) (layer "F.Cu") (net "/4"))
 (segment (start 139.605 43.375) (end 137.98 45) (width 0.25) (layer "F.Cu") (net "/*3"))
 (segment (start 150.055 43.375) (end 139.605 43.375) (width 0.25) (layer "F.Cu") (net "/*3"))
 (segment (start 155.88 49.2) (end 150.055 43.375) (width 0.25) (layer "F.Cu") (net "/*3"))
 (segment (start 138.11 44.87) (end 137.98 45) (width 0.25) (layer "F.Cu") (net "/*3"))
 (segment (start 141.42 45) (end 141.42 45.58) (width 0.25) (layer "F.Cu") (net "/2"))
 (segment (start 158.42 49.2) (end 152.47 43.25) (width 0.25) (layer "B.Cu") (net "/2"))
 (segment (start 152.47 43.25) (end 142.27 43.25) (width 0.25) (layer "B.Cu") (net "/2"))
 (segment (start 142.27 43.25) (end 140.52 45) (width 0.25) (layer "B.Cu") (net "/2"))
 (segment (start 141.25 54.25) (end 143.96 51.54) (width 0.25) (layer "F.Cu") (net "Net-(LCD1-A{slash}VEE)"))
 (segment (start 143.96 51.54) (end 143.06 50.64) (width 0.25) (layer "F.Cu") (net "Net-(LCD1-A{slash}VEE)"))
 (segment (start 143.06 50.64) (end 143.06 45) (width 0.25) (layer "F.Cu") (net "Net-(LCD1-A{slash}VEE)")))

